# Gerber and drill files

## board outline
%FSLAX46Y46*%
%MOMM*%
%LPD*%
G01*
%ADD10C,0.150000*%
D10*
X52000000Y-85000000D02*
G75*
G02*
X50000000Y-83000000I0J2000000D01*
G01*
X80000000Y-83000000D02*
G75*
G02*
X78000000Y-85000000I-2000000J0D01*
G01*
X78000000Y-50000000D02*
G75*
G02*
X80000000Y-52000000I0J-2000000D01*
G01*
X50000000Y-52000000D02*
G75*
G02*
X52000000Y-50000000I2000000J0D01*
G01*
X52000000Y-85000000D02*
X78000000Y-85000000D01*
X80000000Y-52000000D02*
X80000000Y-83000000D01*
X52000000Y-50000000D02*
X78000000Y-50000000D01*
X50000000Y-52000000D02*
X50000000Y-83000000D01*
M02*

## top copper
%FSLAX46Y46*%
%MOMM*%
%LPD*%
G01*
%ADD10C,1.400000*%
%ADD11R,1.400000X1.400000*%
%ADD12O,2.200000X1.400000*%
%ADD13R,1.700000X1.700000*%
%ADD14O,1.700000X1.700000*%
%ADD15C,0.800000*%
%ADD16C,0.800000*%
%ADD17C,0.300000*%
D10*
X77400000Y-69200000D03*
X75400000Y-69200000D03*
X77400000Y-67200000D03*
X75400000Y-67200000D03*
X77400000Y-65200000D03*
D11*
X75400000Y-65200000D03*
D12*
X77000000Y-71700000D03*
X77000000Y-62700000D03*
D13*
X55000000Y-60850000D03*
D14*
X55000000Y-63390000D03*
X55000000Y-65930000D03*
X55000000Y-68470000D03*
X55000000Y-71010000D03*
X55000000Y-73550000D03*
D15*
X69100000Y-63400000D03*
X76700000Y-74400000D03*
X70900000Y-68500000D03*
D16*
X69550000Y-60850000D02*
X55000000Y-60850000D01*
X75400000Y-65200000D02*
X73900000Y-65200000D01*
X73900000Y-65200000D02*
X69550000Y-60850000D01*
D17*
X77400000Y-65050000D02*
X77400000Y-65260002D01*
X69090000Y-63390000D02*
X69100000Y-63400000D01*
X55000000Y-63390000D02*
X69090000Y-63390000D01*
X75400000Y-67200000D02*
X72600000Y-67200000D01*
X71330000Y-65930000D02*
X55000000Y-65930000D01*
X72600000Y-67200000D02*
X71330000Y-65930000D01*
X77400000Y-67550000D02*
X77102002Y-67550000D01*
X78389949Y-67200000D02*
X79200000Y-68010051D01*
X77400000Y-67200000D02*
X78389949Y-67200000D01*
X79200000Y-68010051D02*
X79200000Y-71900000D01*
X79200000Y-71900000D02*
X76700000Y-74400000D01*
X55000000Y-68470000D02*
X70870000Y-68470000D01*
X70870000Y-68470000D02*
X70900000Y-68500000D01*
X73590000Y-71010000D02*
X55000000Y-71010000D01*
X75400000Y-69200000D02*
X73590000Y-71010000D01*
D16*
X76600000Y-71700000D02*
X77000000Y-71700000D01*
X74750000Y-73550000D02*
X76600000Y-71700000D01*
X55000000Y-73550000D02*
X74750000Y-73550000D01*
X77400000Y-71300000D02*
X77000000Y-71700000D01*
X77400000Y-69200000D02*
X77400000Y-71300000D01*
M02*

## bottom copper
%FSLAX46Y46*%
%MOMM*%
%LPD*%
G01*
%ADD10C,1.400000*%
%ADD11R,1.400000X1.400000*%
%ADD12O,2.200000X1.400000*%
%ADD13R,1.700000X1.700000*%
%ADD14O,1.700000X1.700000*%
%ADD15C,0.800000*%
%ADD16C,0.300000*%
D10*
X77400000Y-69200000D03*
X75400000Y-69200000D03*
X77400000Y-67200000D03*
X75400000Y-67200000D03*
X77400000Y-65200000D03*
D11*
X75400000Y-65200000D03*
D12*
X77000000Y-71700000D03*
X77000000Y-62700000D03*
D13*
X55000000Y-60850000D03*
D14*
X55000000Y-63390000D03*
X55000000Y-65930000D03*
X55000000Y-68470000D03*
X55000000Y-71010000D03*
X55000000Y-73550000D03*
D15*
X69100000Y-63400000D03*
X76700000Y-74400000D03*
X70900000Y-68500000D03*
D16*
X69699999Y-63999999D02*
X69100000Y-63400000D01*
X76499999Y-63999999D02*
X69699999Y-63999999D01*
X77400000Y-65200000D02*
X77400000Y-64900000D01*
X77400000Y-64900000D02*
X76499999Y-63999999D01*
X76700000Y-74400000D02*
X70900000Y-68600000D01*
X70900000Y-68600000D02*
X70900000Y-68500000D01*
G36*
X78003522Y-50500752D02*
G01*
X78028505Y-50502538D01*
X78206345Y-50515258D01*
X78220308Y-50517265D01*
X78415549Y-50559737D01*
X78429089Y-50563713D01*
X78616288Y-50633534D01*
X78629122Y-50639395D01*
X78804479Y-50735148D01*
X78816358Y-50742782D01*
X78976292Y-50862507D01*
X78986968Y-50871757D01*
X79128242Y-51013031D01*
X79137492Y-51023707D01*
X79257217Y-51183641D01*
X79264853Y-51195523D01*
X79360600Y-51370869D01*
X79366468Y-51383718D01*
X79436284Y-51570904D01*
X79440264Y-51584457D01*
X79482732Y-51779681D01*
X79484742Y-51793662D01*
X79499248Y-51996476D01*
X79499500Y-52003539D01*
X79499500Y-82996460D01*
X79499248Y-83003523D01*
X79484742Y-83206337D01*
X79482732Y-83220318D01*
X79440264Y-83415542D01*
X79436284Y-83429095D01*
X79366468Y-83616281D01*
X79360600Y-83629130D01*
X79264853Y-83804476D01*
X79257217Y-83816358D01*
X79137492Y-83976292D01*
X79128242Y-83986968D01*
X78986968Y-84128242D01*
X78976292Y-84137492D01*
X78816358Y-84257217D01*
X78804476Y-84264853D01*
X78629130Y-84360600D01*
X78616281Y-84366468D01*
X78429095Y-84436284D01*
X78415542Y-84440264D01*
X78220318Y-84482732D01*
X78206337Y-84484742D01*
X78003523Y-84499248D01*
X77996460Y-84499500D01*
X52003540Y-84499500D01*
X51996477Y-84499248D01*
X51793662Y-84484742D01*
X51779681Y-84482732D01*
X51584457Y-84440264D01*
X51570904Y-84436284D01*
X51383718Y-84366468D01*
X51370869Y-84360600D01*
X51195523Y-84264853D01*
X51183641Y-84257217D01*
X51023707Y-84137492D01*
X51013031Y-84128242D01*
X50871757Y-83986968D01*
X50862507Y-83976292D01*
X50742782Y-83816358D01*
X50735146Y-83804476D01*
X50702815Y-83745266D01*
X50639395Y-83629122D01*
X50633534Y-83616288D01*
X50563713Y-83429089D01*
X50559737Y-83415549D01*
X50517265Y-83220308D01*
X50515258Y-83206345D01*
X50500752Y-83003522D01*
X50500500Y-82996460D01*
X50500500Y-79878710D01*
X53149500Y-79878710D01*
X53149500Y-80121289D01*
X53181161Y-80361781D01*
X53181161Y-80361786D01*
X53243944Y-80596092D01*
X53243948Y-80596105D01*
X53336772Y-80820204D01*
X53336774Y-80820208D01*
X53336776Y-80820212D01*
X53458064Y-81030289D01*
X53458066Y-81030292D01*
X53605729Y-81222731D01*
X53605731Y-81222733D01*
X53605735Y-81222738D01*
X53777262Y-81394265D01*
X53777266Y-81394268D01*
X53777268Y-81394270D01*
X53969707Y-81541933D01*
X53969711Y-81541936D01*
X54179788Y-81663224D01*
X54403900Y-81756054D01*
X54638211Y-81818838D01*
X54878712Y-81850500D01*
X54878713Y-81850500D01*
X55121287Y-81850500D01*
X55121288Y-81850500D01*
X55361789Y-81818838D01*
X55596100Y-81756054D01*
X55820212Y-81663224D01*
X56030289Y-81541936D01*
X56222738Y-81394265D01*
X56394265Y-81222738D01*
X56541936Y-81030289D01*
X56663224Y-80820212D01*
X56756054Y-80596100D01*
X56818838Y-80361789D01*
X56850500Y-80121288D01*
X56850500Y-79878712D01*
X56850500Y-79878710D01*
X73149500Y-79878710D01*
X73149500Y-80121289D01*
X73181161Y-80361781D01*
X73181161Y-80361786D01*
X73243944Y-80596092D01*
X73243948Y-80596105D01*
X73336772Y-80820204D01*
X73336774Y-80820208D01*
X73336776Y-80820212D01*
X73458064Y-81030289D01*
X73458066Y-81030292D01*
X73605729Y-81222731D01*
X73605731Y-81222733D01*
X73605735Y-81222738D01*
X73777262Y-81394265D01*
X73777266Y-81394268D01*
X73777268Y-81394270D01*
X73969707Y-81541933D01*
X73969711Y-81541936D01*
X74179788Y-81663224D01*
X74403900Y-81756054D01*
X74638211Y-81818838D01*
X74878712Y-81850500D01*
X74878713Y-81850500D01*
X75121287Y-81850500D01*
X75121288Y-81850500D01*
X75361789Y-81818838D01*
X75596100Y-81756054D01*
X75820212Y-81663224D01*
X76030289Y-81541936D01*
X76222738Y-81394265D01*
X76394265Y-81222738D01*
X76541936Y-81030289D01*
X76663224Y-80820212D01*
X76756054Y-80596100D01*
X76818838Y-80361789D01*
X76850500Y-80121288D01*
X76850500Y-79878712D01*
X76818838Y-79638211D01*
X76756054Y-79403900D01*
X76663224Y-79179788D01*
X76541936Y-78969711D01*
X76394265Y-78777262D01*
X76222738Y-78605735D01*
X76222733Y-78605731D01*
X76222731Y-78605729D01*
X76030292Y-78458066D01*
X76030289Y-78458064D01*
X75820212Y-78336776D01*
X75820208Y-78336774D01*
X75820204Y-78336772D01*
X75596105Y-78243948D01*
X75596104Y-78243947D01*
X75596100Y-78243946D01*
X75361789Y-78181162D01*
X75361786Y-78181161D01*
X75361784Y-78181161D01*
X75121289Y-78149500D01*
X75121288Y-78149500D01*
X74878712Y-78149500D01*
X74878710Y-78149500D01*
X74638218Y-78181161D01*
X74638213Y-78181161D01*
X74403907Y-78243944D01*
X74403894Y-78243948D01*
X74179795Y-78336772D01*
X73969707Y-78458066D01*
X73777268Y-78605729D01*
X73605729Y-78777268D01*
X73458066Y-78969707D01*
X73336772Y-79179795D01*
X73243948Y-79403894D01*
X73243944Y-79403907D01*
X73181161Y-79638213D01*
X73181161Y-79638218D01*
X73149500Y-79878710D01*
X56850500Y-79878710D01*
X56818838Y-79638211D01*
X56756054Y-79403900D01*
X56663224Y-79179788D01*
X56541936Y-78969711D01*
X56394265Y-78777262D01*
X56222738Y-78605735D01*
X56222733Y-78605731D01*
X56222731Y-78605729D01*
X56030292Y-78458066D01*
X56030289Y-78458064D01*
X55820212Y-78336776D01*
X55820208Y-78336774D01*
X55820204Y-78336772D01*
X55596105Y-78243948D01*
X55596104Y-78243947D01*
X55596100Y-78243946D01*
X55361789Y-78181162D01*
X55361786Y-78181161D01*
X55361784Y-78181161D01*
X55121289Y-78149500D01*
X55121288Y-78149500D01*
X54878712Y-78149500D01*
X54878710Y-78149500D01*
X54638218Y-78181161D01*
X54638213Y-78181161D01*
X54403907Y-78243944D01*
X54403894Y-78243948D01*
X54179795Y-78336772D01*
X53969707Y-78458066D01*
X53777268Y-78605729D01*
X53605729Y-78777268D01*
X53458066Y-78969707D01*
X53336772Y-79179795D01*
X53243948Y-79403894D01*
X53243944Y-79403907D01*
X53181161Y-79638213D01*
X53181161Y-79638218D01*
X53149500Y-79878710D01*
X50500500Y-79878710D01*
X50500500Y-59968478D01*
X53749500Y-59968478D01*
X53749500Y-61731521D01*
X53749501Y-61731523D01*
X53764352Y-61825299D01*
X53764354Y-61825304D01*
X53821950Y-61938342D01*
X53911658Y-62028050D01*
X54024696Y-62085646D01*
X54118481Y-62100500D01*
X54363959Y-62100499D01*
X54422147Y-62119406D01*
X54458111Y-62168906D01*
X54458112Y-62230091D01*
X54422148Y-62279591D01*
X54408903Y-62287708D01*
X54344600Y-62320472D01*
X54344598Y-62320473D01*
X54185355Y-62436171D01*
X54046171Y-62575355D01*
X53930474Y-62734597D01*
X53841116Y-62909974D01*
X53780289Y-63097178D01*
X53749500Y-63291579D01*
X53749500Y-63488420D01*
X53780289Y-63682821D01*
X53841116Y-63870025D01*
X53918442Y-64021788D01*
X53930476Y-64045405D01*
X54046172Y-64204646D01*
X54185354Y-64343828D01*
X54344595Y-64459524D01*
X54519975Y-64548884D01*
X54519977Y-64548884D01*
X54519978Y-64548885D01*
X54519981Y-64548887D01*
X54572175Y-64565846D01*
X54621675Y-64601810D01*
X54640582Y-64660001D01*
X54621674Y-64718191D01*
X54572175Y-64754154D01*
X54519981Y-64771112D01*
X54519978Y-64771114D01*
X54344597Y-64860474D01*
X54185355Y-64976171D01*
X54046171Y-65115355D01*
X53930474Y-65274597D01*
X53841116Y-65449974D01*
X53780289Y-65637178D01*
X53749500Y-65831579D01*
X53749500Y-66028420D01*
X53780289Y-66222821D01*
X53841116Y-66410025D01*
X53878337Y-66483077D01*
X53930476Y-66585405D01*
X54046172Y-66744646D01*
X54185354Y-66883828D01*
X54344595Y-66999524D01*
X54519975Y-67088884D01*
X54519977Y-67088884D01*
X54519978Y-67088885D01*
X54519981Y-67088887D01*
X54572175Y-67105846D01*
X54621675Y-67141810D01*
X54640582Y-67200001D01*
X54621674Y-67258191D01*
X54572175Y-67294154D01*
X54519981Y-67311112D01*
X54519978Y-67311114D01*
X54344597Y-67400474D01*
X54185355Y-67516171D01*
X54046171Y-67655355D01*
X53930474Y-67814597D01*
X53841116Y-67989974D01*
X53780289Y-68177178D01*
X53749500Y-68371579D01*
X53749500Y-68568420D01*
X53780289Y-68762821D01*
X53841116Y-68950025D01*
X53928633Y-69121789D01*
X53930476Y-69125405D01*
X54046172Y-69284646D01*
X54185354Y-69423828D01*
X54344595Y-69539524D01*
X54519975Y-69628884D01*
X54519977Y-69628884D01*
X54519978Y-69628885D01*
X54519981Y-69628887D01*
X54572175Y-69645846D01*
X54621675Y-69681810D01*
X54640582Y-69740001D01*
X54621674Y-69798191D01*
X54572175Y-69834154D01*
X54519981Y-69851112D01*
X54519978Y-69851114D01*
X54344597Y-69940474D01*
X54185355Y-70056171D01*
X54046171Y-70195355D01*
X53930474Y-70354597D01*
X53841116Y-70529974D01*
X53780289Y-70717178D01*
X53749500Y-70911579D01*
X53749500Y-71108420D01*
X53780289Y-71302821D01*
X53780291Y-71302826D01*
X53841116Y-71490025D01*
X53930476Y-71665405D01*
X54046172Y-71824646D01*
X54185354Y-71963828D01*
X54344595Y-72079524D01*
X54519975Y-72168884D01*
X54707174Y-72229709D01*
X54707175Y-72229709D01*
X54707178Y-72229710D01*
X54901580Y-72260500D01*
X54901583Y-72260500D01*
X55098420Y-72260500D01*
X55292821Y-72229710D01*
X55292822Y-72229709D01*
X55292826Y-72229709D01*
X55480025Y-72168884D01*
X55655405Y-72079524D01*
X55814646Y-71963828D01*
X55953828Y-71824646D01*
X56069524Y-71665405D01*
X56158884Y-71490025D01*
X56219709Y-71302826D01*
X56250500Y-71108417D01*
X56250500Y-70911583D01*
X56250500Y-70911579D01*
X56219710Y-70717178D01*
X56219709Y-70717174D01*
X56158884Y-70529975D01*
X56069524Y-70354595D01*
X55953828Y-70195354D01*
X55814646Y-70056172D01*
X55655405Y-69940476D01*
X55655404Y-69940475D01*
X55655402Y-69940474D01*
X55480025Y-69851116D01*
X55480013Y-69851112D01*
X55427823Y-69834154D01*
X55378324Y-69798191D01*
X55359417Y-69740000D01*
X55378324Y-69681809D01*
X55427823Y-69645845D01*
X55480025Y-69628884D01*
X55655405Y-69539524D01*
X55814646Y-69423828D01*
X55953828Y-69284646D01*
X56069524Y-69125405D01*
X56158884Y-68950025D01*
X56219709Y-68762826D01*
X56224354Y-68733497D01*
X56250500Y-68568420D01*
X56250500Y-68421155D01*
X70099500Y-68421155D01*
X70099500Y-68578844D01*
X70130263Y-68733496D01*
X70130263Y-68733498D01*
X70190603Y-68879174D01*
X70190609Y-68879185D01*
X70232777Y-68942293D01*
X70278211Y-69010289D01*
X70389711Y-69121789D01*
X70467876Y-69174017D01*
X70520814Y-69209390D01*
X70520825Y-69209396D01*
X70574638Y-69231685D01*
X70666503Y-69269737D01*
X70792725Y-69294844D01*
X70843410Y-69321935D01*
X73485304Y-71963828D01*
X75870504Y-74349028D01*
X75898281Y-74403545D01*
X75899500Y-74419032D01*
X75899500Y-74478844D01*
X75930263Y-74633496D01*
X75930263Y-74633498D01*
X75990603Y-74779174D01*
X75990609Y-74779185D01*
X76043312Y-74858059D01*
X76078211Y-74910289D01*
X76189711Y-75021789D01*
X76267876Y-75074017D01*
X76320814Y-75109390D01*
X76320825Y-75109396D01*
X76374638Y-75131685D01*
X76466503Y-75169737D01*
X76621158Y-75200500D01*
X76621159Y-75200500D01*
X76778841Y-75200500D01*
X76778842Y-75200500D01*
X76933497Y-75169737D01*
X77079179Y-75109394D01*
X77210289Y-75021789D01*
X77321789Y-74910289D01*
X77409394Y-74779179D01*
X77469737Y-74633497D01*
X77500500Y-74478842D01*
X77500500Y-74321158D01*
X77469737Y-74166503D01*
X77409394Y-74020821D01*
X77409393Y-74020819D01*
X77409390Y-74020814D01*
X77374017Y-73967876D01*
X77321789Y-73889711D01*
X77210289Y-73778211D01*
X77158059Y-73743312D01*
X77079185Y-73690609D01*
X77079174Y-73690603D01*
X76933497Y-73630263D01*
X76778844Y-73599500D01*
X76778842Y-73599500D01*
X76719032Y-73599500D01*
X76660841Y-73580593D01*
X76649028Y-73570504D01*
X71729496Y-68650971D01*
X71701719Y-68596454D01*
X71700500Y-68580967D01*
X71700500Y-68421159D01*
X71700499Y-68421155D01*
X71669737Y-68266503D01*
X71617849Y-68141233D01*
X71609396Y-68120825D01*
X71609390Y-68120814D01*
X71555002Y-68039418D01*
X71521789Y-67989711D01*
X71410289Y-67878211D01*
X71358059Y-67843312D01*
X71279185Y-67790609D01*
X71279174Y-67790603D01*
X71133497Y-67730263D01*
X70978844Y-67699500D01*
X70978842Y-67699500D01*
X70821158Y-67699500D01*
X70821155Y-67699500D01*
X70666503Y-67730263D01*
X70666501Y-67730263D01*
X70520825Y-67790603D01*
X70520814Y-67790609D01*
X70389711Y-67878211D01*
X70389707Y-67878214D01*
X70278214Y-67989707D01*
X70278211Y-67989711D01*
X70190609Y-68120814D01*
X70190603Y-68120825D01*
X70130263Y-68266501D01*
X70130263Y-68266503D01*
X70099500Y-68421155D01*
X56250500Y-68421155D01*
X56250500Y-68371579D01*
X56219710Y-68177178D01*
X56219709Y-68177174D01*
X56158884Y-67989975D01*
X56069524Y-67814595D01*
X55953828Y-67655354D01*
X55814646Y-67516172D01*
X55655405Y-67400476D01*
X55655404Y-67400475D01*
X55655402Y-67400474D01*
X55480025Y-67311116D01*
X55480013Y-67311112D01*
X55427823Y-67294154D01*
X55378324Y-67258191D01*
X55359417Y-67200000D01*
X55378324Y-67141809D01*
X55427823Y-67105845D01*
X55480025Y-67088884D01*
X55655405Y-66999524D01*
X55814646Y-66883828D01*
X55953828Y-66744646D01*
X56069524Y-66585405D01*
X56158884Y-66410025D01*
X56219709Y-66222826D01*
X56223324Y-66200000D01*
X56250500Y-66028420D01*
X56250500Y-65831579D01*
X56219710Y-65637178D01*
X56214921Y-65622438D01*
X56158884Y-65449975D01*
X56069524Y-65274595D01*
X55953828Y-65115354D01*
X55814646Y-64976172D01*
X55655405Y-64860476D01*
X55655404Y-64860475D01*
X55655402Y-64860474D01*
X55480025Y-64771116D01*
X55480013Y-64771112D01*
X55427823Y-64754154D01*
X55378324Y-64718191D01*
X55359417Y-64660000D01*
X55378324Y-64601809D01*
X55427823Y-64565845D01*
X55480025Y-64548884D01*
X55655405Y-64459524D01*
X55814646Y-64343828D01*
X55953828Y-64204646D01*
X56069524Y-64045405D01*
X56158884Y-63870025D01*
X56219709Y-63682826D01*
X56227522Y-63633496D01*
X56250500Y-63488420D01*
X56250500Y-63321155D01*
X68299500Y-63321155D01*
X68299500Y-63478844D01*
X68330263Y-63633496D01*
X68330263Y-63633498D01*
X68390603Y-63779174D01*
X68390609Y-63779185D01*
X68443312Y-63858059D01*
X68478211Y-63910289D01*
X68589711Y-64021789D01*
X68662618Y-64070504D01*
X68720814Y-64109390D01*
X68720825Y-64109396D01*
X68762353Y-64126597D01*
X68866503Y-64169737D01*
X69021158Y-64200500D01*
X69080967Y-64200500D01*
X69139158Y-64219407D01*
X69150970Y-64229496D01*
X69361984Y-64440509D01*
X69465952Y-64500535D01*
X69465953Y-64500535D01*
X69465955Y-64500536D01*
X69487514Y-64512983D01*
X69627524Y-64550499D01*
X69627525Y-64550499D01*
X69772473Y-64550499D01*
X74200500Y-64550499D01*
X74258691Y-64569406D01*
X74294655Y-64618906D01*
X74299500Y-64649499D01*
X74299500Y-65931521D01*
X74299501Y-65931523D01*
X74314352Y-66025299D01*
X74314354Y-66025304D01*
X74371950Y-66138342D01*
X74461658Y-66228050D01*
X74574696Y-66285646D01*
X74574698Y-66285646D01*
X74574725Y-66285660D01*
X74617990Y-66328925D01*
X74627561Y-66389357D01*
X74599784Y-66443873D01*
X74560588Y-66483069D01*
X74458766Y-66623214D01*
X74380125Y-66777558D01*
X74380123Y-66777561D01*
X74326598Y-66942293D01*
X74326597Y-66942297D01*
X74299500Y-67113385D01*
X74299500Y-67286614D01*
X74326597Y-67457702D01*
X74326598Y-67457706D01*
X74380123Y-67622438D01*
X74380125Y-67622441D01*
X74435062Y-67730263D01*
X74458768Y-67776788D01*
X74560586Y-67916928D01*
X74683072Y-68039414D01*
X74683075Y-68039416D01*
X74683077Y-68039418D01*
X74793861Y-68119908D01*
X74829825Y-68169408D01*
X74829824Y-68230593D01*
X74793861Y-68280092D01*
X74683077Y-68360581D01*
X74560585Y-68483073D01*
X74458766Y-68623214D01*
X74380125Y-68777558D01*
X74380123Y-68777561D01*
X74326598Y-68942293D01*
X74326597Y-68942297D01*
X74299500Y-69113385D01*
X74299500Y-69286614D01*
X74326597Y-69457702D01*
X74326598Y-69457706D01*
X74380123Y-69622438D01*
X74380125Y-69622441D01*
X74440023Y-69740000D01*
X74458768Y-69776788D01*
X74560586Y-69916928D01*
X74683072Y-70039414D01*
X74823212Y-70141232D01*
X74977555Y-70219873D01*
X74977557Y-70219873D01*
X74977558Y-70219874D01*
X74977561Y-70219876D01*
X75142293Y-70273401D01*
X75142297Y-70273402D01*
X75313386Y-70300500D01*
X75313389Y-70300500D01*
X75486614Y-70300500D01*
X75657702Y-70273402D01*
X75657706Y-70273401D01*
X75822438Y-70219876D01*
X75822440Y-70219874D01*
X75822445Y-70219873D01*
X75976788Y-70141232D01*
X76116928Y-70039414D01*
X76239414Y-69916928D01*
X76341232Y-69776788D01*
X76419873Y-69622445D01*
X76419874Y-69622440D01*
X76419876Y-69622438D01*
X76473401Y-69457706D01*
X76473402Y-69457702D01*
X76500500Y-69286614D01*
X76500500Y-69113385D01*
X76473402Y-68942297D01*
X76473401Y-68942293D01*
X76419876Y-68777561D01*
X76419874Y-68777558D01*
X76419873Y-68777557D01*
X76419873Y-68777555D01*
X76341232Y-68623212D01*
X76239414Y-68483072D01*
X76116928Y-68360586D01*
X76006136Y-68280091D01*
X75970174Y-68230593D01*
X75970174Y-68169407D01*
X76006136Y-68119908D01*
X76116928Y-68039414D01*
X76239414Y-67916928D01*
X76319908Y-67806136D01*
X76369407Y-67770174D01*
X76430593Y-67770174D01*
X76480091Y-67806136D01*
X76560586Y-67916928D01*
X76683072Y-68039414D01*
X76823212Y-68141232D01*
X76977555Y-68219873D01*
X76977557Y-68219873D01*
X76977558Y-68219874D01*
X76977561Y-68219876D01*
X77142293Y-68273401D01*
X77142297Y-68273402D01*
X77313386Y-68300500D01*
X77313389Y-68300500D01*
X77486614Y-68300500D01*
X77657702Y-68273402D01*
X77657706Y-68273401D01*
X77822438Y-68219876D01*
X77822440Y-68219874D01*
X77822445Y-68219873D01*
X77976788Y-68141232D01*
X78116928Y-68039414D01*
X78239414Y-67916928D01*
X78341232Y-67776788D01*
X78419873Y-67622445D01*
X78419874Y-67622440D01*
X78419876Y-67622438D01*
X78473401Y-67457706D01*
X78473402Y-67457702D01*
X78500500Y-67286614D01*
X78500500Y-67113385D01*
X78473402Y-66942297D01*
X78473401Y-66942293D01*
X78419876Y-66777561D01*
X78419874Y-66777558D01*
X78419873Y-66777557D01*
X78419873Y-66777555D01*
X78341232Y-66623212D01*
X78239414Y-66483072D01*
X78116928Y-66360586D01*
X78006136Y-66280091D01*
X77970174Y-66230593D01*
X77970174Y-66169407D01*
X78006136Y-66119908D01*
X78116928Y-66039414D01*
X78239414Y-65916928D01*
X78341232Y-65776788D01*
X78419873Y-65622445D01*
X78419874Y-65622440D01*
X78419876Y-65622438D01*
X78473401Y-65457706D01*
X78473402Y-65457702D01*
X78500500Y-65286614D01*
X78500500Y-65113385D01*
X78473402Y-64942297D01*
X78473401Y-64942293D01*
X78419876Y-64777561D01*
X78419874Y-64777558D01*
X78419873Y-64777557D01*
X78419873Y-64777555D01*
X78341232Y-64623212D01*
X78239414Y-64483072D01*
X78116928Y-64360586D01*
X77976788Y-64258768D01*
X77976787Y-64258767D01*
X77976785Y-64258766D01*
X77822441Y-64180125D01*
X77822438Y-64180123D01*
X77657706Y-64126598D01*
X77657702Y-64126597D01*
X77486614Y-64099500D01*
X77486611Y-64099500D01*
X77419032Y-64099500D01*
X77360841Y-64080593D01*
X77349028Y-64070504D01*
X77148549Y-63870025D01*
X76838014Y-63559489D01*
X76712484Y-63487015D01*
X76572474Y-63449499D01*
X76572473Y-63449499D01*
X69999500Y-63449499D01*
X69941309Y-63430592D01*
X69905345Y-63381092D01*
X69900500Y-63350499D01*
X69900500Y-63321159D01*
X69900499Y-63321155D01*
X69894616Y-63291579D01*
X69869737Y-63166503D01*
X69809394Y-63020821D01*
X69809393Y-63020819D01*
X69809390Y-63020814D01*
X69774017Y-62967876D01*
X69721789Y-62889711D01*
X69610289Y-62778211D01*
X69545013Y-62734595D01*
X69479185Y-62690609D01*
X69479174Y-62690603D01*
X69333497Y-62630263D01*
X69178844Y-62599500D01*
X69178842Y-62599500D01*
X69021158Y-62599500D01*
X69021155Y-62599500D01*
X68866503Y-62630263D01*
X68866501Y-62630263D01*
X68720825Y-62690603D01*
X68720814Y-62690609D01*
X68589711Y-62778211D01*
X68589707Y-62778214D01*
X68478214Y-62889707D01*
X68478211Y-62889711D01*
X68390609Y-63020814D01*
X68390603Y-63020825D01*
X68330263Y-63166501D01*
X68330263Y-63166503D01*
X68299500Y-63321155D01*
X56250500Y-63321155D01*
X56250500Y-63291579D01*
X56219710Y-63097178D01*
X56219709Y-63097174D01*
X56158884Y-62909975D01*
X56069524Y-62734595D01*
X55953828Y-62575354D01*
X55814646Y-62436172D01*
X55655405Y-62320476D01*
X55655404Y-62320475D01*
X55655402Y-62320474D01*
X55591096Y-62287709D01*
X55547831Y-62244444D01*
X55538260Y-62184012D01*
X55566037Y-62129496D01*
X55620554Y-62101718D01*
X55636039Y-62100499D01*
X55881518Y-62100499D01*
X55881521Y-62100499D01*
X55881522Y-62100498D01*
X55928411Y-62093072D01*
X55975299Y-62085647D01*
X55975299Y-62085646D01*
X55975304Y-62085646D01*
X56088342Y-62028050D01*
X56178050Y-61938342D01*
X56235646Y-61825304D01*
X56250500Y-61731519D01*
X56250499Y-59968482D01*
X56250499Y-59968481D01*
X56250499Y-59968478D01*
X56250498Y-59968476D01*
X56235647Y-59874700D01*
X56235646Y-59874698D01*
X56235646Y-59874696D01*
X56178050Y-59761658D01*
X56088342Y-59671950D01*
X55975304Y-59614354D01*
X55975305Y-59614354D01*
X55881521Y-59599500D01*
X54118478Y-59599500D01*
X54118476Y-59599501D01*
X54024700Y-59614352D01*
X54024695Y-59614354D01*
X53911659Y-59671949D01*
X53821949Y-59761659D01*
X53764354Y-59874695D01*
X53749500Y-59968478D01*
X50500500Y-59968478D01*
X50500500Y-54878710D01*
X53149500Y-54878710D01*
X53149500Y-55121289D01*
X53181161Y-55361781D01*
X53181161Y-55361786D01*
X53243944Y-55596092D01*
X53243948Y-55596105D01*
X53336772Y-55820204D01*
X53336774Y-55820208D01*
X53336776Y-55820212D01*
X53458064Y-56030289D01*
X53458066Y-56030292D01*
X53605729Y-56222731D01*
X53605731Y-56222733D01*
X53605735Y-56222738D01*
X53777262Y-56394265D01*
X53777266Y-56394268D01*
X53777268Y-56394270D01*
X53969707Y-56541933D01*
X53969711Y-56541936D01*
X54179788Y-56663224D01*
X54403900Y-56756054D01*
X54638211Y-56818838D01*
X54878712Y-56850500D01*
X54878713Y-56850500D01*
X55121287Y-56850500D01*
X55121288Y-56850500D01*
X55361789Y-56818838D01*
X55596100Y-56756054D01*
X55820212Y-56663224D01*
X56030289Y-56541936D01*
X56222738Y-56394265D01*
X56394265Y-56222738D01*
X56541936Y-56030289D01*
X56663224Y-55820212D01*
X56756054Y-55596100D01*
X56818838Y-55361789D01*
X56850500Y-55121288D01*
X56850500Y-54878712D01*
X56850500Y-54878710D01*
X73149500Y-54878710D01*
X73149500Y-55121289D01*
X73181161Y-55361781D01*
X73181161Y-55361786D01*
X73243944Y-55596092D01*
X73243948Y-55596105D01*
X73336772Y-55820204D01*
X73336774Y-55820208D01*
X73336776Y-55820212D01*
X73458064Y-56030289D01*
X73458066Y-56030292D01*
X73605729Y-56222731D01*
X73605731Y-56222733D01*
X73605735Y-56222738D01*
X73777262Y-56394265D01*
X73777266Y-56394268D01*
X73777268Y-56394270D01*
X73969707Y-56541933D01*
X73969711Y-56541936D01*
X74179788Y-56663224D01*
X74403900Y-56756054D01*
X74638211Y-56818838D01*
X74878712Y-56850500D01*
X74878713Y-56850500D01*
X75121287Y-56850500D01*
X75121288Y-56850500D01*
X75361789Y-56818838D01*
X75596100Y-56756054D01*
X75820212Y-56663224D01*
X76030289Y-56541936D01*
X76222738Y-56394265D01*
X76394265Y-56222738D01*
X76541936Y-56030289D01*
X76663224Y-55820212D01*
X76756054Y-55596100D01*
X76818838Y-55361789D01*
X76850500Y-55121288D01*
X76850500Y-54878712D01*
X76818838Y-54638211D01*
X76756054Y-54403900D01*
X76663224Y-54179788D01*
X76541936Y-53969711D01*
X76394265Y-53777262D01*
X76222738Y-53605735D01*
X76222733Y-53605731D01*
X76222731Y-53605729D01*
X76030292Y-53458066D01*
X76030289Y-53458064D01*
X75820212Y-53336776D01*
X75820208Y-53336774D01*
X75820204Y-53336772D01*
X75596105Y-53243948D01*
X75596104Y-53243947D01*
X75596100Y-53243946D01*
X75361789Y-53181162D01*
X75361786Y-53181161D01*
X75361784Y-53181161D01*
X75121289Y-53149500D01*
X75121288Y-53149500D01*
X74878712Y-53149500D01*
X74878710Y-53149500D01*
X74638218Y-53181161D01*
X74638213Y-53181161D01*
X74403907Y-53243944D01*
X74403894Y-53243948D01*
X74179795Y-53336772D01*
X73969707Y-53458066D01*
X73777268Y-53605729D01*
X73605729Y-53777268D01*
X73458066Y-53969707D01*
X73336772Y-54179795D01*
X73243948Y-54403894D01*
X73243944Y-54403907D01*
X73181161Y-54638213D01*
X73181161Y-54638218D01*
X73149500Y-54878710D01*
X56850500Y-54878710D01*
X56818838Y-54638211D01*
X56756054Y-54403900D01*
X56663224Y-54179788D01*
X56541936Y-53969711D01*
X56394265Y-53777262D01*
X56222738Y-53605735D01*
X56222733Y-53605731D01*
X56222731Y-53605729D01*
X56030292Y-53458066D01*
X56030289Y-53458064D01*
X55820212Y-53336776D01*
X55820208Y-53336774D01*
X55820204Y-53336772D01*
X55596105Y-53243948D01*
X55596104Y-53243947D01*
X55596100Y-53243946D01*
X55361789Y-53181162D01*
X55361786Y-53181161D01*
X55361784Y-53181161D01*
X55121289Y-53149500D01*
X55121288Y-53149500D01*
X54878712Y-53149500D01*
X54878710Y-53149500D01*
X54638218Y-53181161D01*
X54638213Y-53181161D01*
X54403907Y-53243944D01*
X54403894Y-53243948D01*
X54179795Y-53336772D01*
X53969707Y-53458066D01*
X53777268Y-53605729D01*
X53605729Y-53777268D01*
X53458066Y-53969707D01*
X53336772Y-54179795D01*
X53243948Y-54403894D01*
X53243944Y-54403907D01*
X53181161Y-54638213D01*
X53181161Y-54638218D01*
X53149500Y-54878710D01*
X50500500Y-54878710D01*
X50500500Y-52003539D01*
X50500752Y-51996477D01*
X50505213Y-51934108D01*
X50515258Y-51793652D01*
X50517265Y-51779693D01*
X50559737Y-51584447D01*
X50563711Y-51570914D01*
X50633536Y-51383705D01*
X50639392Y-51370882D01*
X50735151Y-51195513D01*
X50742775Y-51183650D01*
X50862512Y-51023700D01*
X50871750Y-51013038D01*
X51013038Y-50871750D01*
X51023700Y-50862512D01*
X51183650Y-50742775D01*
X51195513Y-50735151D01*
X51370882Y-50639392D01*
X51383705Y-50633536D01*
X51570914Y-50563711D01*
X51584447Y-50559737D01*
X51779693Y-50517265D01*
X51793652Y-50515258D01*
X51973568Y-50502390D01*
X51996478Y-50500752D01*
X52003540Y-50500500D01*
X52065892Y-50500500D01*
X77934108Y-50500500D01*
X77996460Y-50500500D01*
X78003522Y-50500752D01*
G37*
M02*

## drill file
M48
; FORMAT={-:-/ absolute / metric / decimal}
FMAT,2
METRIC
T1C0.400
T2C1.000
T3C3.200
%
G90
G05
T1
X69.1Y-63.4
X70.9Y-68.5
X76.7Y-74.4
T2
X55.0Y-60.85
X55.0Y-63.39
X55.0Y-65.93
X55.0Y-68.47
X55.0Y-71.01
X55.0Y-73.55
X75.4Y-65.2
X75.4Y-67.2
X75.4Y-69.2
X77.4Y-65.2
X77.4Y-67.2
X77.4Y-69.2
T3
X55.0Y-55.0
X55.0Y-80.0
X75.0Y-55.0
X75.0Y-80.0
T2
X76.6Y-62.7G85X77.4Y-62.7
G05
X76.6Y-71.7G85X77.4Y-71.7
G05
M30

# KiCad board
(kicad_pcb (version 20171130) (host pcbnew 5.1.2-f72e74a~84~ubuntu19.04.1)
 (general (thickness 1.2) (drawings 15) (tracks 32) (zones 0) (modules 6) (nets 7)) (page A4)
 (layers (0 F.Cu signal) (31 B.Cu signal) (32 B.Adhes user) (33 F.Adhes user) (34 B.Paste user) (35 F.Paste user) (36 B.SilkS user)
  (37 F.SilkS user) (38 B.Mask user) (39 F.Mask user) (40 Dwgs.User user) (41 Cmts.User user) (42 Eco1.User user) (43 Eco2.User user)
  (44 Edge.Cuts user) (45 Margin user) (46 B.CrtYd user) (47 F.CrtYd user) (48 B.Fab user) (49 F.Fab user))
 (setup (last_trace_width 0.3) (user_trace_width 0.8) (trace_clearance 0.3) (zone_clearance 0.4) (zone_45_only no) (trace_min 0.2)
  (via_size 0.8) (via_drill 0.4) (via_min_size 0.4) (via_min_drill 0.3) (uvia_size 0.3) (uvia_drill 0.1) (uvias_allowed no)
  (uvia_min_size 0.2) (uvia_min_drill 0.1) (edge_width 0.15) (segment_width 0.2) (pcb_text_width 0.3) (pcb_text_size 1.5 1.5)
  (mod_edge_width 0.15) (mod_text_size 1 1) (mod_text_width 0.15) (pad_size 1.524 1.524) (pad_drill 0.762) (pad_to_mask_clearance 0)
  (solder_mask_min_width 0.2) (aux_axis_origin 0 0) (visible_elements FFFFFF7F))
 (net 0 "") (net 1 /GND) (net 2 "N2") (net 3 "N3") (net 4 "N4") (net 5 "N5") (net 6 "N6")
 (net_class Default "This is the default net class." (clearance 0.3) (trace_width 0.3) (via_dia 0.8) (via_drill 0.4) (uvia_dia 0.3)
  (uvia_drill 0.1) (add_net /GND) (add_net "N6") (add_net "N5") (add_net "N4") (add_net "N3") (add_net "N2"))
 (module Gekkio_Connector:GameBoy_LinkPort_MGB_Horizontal (layer F.Cu) (at 75.4 65.2)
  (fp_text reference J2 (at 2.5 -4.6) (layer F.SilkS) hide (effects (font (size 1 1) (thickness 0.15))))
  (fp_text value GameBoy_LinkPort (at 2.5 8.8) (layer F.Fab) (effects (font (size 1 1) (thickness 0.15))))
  (pad 6 thru_hole circle (at 2 4) (size 1.4 1.4) (drill 1) (layers *.Cu *.Mask) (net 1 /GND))
  (pad 5 thru_hole circle (at 0 4) (size 1.4 1.4) (drill 1) (layers *.Cu *.Mask) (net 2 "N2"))
  (pad 4 thru_hole circle (at 2 2) (size 1.4 1.4) (drill 1) (layers *.Cu *.Mask) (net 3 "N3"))
  (pad 3 thru_hole circle (at 0 2) (size 1.4 1.4) (drill 1) (layers *.Cu *.Mask) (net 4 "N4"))
  (pad 2 thru_hole circle (at 2 0) (size 1.4 1.4) (drill 1) (layers *.Cu *.Mask) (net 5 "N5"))
  (pad 1 thru_hole rect (at 0 0) (size 1.4 1.4) (drill 1) (layers *.Cu *.Mask) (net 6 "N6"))
  (pad SH thru_hole oval (at 1.6 6.5 90) (size 1.4 2.2) (drill oval 1 1.8) (layers *.Cu *.Mask) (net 1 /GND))
  (pad SH thru_hole oval (at 1.6 -2.5 90) (size 1.4 2.2) (drill oval 1 1.8) (layers *.Cu *.Mask) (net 1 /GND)))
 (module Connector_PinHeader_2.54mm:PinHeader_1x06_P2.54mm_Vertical (layer F.Cu) (at 55 60.85)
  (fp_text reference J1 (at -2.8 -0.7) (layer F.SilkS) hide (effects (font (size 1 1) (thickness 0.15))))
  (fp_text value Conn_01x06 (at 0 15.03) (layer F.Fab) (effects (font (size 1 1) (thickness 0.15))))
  (pad 1 thru_hole rect (at 0 0) (size 1.7 1.7) (drill 1) (layers *.Cu *.Mask) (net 6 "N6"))
  (pad 2 thru_hole oval (at 0 2.54) (size 1.7 1.7) (drill 1) (layers *.Cu *.Mask) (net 5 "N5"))
  (pad 3 thru_hole oval (at 0 5.08) (size 1.7 1.7) (drill 1) (layers *.Cu *.Mask) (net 4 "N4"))
  (pad 4 thru_hole oval (at 0 7.62) (size 1.7 1.7) (drill 1) (layers *.Cu *.Mask) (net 3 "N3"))
  (pad 5 thru_hole oval (at 0 10.16) (size 1.7 1.7) (drill 1) (layers *.Cu *.Mask) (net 2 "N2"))
  (pad 6 thru_hole oval (at 0 12.7) (size 1.7 1.7) (drill 1) (layers *.Cu *.Mask) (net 1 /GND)))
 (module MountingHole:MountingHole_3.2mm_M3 (layer F.Cu) (at 75 80)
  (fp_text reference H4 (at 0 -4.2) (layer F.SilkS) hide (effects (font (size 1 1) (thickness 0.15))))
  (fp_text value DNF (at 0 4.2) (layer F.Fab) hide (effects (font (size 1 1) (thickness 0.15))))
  (pad 1 np_thru_hole circle (at 0 0) (size 3.2 3.2) (drill 3.2) (layers *.Cu *.Mask)))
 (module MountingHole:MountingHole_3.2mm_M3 (layer F.Cu) (at 75 55)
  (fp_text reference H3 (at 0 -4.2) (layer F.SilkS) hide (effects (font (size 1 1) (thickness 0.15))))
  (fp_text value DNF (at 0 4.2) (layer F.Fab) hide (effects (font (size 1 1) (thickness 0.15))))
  (pad 1 np_thru_hole circle (at 0 0) (size 3.2 3.2) (drill 3.2) (layers *.Cu *.Mask)))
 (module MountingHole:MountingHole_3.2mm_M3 (layer F.Cu) (at 55 80)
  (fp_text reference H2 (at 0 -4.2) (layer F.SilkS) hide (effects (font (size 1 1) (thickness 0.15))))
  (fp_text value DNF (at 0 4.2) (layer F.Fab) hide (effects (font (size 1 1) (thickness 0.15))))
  (pad 1 np_thru_hole circle (at 0 0) (size 3.2 3.2) (drill 3.2) (layers *.Cu *.Mask)))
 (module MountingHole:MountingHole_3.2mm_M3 (layer F.Cu) (at 55 55)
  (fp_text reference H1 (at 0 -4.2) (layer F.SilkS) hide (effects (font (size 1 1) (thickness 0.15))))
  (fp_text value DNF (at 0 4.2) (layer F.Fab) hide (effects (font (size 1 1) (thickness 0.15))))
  (pad 1 np_thru_hole circle (at 0 0) (size 3.2 3.2) (drill 3.2) (layers *.Cu *.Mask)))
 (gr_arc (start 52 83) (end 50 83) (angle -90) (layer Edge.Cuts) (width 0.15))
 (gr_arc (start 78 83) (end 78 85) (angle -90) (layer Edge.Cuts) (width 0.15))
 (gr_arc (start 78 52) (end 80 52) (angle -90) (layer Edge.Cuts) (width 0.15))
 (gr_arc (start 52 52) (end 52 50) (angle -90) (layer Edge.Cuts) (width 0.15))
 (gr_line (start 52 85) (end 78 85) (layer Edge.Cuts) (width 0.15))
 (gr_line (start 80 52) (end 80 83) (layer Edge.Cuts) (width 0.15))
 (gr_line (start 52 50) (end 78 50) (layer Edge.Cuts) (width 0.15))
 (gr_line (start 50 52) (end 50 83) (layer Edge.Cuts) (width 0.15))
 (segment (start 69.55 60.85) (end 55 60.85) (width 0.8) (layer F.Cu) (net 6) (status 20))
 (segment (start 75.4 65.2) (end 73.9 65.2) (width 0.8) (layer F.Cu) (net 6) (status 10))
 (segment (start 73.9 65.2) (end 69.55 60.85) (width 0.8) (layer F.Cu) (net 6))
 (segment (start 77.4 65.05) (end 77.4 65.260002) (width 0.3) (layer F.Cu) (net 5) (status 30))
 (segment (start 69.09 63.39) (end 69.1 63.4) (width 0.3) (layer F.Cu) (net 5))
 (segment (start 55 63.39) (end 69.09 63.39) (width 0.3) (layer F.Cu) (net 5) (status 10))
 (via (at 69.1 63.4) (size 0.8) (drill 0.4) (layers F.Cu B.Cu) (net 5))
 (segment (start 69.699999 63.999999) (end 69.1 63.4) (width 0.3) (layer B.Cu) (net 5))
 (segment (start 76.499999 63.999999) (end 69.699999 63.999999) (width 0.3) (layer B.Cu) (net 5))
 (segment (start 77.4 65.2) (end 77.4 64.9) (width 0.3) (layer B.Cu) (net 5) (status 30))
 (segment (start 77.4 64.9) (end 76.499999 63.999999) (width 0.3) (layer B.Cu) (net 5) (status 10))
 (segment (start 75.4 67.2) (end 72.6 67.2) (width 0.3) (layer F.Cu) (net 4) (status 10))
 (segment (start 71.33 65.93) (end 55 65.93) (width 0.3) (layer F.Cu) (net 4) (status 20))
 (segment (start 72.6 67.2) (end 71.33 65.93) (width 0.3) (layer F.Cu) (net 4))
 (segment (start 77.4 67.55) (end 77.102002 67.55) (width 0.3) (layer F.Cu) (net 3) (status 30))
 (segment (start 78.389949 67.2) (end 79.2 68.010051) (width 0.3) (layer F.Cu) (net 3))
 (segment (start 77.4 67.2) (end 78.389949 67.2) (width 0.3) (layer F.Cu) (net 3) (status 10))
 (via (at 76.7 74.4) (size 0.8) (drill 0.4) (layers F.Cu B.Cu) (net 3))
 (segment (start 79.2 68.010051) (end 79.2 71.9) (width 0.3) (layer F.Cu) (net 3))
 (segment (start 79.2 71.9) (end 76.7 74.4) (width 0.3) (layer F.Cu) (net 3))
 (segment (start 76.7 74.4) (end 70.9 68.6) (width 0.3) (layer B.Cu) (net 3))
 (segment (start 70.9 68.6) (end 70.9 68.5) (width 0.3) (layer B.Cu) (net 3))
 (via (at 70.9 68.5) (size 0.8) (drill 0.4) (layers F.Cu B.Cu) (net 3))
 (segment (start 55 68.47) (end 70.87 68.47) (width 0.3) (layer F.Cu) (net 3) (status 10))
 (segment (start 70.87 68.47) (end 70.9 68.5) (width 0.3) (layer F.Cu) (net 3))
 (segment (start 73.59 71.01) (end 55 71.01) (width 0.3) (layer F.Cu) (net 2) (status 20))
 (segment (start 75.4 69.2) (end 73.59 71.01) (width 0.3) (layer F.Cu) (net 2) (status 10))
 (segment (start 76.6 71.7) (end 77 71.7) (width 0.8) (layer F.Cu) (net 1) (status 30))
 (segment (start 74.75 73.55) (end 76.6 71.7) (width 0.8) (layer F.Cu) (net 1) (status 20))
 (segment (start 55 73.55) (end 74.75 73.55) (width 0.8) (layer F.Cu) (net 1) (status 10))
 (segment (start 77.4 71.3) (end 77 71.7) (width 0.8) (layer F.Cu) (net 1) (status 30))
 (segment (start 77.4 69.2) (end 77.4 71.3) (width 0.8) (layer F.Cu) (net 1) (status 30))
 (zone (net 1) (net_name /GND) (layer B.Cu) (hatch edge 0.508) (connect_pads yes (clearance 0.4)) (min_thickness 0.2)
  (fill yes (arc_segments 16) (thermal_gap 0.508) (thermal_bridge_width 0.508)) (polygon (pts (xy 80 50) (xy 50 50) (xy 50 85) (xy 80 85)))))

